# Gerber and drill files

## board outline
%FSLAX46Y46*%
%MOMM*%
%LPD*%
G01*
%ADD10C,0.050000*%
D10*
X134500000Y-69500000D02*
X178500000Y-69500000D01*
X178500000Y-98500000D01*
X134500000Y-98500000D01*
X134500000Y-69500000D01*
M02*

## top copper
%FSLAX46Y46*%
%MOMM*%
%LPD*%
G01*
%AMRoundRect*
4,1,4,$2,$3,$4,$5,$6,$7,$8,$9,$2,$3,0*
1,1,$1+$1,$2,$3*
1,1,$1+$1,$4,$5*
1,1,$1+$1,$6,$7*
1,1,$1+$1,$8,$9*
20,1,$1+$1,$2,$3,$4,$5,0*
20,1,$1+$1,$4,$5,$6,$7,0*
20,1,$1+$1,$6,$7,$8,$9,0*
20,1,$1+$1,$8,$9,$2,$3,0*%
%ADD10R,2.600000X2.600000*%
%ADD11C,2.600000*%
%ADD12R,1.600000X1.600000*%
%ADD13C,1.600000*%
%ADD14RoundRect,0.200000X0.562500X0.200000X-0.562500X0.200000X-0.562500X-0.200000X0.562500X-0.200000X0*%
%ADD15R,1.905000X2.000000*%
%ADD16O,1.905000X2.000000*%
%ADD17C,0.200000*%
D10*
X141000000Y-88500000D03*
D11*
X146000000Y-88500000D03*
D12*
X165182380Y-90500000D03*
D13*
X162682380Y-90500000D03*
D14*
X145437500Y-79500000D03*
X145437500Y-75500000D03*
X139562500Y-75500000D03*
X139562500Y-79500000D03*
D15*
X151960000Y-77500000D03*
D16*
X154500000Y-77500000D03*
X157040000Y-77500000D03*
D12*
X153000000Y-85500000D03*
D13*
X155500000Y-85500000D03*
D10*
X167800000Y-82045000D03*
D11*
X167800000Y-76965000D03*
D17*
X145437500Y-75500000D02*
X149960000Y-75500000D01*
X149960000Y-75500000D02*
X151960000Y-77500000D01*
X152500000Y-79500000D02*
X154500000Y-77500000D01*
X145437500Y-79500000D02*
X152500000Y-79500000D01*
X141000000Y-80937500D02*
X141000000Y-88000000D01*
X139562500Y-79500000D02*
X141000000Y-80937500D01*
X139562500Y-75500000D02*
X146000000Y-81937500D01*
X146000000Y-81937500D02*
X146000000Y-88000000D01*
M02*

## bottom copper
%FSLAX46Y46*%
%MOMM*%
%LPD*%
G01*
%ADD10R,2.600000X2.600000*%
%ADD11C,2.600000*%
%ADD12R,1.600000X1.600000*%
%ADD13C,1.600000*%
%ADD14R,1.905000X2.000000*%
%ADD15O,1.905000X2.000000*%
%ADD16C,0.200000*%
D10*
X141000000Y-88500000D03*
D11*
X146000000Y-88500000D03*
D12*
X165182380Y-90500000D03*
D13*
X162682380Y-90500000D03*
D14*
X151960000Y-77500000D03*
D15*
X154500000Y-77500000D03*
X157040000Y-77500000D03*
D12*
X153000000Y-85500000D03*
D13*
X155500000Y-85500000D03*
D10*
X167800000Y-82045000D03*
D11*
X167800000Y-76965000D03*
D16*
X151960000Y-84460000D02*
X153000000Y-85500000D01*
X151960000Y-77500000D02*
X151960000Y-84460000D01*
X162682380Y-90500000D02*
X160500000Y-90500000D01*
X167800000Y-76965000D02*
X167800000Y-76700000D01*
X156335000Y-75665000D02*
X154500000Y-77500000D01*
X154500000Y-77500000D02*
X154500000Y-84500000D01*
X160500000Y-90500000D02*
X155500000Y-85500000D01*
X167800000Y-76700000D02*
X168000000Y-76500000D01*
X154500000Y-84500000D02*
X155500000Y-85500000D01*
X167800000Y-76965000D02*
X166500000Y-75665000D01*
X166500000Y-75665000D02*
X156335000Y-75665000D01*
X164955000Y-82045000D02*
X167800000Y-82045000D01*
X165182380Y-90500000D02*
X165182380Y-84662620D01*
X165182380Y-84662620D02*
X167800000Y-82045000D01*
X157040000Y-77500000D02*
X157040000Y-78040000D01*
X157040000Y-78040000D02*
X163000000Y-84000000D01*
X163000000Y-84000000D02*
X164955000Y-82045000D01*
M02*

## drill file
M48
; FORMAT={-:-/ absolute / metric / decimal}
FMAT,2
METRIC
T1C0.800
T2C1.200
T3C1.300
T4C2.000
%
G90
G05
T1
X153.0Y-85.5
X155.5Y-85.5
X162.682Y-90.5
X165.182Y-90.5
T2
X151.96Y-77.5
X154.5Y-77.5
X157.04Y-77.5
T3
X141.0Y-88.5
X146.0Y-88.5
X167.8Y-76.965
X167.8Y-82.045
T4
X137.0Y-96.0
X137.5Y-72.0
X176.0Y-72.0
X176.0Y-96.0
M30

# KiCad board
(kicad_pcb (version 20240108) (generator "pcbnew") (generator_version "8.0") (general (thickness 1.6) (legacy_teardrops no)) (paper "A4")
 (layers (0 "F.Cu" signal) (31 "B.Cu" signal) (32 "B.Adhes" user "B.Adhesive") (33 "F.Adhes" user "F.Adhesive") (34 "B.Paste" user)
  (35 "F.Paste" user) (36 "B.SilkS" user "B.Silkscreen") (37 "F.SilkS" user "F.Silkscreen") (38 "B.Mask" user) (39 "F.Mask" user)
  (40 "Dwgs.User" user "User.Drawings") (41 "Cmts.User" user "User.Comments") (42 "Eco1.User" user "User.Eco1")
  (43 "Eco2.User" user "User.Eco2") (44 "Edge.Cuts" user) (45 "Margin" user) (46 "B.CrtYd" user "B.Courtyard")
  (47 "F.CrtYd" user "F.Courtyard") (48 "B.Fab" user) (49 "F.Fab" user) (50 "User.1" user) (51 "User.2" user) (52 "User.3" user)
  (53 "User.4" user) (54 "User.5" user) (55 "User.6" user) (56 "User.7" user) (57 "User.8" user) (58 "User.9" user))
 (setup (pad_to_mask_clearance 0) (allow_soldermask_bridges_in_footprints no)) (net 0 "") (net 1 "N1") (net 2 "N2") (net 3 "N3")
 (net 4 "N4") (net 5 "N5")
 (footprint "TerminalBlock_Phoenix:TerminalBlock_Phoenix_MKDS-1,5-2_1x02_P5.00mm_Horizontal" (layer "F.Cu") (at 141 88.5)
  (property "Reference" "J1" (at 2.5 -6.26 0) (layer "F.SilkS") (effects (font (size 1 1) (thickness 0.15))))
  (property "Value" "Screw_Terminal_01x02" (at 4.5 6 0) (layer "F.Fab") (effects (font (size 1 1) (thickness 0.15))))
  (pad "1" thru_hole rect (at 0 0) (size 2.6 2.6) (drill 1.3) (layers "*.Cu" "*.Mask") (remove_unused_layers no) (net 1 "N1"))
  (pad "2" thru_hole circle (at 5 0) (size 2.6 2.6) (drill 1.3) (layers "*.Cu" "*.Mask") (remove_unused_layers no) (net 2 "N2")))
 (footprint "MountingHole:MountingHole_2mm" (layer "F.Cu") (at 176 72)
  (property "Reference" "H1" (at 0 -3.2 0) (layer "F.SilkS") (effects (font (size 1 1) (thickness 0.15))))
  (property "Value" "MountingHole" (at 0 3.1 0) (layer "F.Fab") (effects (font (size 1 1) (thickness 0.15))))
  (pad "" np_thru_hole circle (at 0 0) (size 2 2) (drill 2) (layers "*.Cu" "*.Mask")))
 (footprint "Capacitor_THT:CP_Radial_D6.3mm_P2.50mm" (layer "F.Cu") (at 165.18238 90.5 180)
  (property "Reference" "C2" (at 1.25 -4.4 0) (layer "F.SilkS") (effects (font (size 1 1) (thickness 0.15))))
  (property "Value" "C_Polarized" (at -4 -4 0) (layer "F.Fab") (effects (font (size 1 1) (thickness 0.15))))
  (pad "1" thru_hole rect (at 0 0 180) (size 1.6 1.6) (drill 0.8) (layers "*.Cu" "*.Mask") (remove_unused_layers no) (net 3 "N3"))
  (pad "2" thru_hole circle (at 2.5 0 180) (size 1.6 1.6) (drill 0.8) (layers "*.Cu" "*.Mask") (remove_unused_layers no) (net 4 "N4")))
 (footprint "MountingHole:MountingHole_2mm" (layer "F.Cu") (at 137 96)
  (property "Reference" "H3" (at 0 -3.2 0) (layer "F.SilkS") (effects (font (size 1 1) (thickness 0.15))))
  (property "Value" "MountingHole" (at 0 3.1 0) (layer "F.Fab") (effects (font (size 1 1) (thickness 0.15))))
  (pad "" np_thru_hole circle (at 0 0) (size 2 2) (drill 2) (layers "*.Cu" "*.Mask")))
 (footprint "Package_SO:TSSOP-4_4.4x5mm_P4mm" (layer "F.Cu") (at 142.5 77.5 180)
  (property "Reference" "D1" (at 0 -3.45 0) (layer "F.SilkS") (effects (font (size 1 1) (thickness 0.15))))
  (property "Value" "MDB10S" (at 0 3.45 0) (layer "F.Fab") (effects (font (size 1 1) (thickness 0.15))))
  (pad "1" smd roundrect (at -2.9375 -2 180) (size 1.525 0.8) (layers "F.Cu" "F.Paste" "F.Mask") (roundrect_rratio 0.25) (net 4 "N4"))
  (pad "2" smd roundrect (at -2.9375 2 180) (size 1.525 0.8) (layers "F.Cu" "F.Paste" "F.Mask") (roundrect_rratio 0.25) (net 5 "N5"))
  (pad "3" smd roundrect (at 2.9375 2 180) (size 1.525 0.8) (layers "F.Cu" "F.Paste" "F.Mask") (roundrect_rratio 0.25) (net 2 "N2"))
  (pad "4" smd roundrect (at 2.9375 -2 180) (size 1.525 0.8) (layers "F.Cu" "F.Paste" "F.Mask") (roundrect_rratio 0.25) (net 1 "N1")))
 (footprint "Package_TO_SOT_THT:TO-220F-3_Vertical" (layer "F.Cu") (at 151.96 77.5)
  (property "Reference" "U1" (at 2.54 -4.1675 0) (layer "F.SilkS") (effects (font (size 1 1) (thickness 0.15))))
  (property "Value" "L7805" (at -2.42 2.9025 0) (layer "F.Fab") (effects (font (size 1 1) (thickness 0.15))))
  (pad "1" thru_hole rect (at 0 0) (size 1.905 2) (drill 1.2) (layers "*.Cu" "*.Mask") (remove_unused_layers no) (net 5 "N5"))
  (pad "2" thru_hole oval (at 2.54 0) (size 1.905 2) (drill 1.2) (layers "*.Cu" "*.Mask") (remove_unused_layers no) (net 4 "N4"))
  (pad "3" thru_hole oval (at 5.08 0) (size 1.905 2) (drill 1.2) (layers "*.Cu" "*.Mask") (remove_unused_layers no) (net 3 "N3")))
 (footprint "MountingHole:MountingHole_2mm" (layer "F.Cu") (at 176 96)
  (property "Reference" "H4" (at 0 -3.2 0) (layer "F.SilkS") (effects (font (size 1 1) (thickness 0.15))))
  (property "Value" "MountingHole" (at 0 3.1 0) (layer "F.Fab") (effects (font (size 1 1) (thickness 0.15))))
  (pad "" np_thru_hole circle (at 0 0) (size 2 2) (drill 2) (layers "*.Cu" "*.Mask")))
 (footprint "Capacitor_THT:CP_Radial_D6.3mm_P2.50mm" (layer "F.Cu") (at 153 85.5)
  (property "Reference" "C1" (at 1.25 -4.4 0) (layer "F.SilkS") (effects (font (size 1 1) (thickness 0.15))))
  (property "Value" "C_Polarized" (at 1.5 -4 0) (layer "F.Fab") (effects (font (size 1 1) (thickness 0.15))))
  (pad "1" thru_hole rect (at 0 0) (size 1.6 1.6) (drill 0.8) (layers "*.Cu" "*.Mask") (remove_unused_layers no) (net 5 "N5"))
  (pad "2" thru_hole circle (at 2.5 0) (size 1.6 1.6) (drill 0.8) (layers "*.Cu" "*.Mask") (remove_unused_layers no) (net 4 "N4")))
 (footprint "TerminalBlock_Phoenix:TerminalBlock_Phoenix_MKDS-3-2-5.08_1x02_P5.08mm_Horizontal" (layer "F.Cu") (at 167.8 82.045 90)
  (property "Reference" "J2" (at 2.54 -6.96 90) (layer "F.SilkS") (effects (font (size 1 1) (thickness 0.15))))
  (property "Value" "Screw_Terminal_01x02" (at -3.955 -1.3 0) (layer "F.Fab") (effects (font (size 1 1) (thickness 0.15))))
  (pad "1" thru_hole rect (at 0 0 90) (size 2.6 2.6) (drill 1.3) (layers "*.Cu" "*.Mask") (remove_unused_layers no) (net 3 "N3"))
  (pad "2" thru_hole circle (at 5.08 0 90) (size 2.6 2.6) (drill 1.3) (layers "*.Cu" "*.Mask") (remove_unused_layers no) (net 4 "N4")))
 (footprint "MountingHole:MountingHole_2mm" (layer "F.Cu") (at 137.5 72)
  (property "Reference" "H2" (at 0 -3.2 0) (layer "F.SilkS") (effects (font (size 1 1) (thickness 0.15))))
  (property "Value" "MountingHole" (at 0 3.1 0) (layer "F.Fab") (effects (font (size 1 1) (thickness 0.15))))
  (pad "" np_thru_hole circle (at 0 0) (size 2 2) (drill 2) (layers "*.Cu" "*.Mask")))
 (gr_rect (start 134.5 69.5) (end 178.5 98.5) (stroke (width 0.05) (type default)) (fill none) (layer "Edge.Cuts"))
 (segment (start 145.4375 75.5) (end 149.96 75.5) (width 0.2) (layer "F.Cu") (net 5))
 (segment (start 149.96 75.5) (end 151.96 77.5) (width 0.2) (layer "F.Cu") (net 5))
 (segment (start 151.96 84.46) (end 153 85.5) (width 0.2) (layer "B.Cu") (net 5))
 (segment (start 151.96 77.5) (end 151.96 84.46) (width 0.2) (layer "B.Cu") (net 5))
 (segment (start 152.5 79.5) (end 154.5 77.5) (width 0.2) (layer "F.Cu") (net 4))
 (segment (start 145.4375 79.5) (end 152.5 79.5) (width 0.2) (layer "F.Cu") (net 4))
 (segment (start 162.68238 90.5) (end 160.5 90.5) (width 0.2) (layer "B.Cu") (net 4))
 (segment (start 167.8 76.965) (end 167.8 76.7) (width 0.2) (layer "B.Cu") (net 4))
 (segment (start 156.335 75.665) (end 154.5 77.5) (width 0.2) (layer "B.Cu") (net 4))
 (segment (start 154.5 77.5) (end 154.5 84.5) (width 0.2) (layer "B.Cu") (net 4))
 (segment (start 160.5 90.5) (end 155.5 85.5) (width 0.2) (layer "B.Cu") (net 4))
 (segment (start 167.8 76.7) (end 168 76.5) (width 0.2) (layer "B.Cu") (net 4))
 (segment (start 154.5 84.5) (end 155.5 85.5) (width 0.2) (layer "B.Cu") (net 4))
 (segment (start 167.8 76.965) (end 166.5 75.665) (width 0.2) (layer "B.Cu") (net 4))
 (segment (start 166.5 75.665) (end 156.335 75.665) (width 0.2) (layer "B.Cu") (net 4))
 (segment (start 141 80.9375) (end 141 88) (width 0.2) (layer "F.Cu") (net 1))
 (segment (start 139.5625 79.5) (end 141 80.9375) (width 0.2) (layer "F.Cu") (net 1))
 (segment (start 139.5625 75.5) (end 146 81.9375) (width 0.2) (layer "F.Cu") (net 2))
 (segment (start 146 81.9375) (end 146 88) (width 0.2) (layer "F.Cu") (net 2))
 (segment (start 164.955 82.045) (end 167.8 82.045) (width 0.2) (layer "B.Cu") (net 3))
 (segment (start 165.18238 90.5) (end 165.18238 84.66262) (width 0.2) (layer "B.Cu") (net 3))
 (segment (start 165.18238 84.66262) (end 167.8 82.045) (width 0.2) (layer "B.Cu") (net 3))
 (segment (start 157.04 77.5) (end 157.04 78.04) (width 0.2) (layer "B.Cu") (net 3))
 (segment (start 157.04 78.04) (end 163 84) (width 0.2) (layer "B.Cu") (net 3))
 (segment (start 163 84) (end 164.955 82.045) (width 0.2) (layer "B.Cu") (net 3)))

